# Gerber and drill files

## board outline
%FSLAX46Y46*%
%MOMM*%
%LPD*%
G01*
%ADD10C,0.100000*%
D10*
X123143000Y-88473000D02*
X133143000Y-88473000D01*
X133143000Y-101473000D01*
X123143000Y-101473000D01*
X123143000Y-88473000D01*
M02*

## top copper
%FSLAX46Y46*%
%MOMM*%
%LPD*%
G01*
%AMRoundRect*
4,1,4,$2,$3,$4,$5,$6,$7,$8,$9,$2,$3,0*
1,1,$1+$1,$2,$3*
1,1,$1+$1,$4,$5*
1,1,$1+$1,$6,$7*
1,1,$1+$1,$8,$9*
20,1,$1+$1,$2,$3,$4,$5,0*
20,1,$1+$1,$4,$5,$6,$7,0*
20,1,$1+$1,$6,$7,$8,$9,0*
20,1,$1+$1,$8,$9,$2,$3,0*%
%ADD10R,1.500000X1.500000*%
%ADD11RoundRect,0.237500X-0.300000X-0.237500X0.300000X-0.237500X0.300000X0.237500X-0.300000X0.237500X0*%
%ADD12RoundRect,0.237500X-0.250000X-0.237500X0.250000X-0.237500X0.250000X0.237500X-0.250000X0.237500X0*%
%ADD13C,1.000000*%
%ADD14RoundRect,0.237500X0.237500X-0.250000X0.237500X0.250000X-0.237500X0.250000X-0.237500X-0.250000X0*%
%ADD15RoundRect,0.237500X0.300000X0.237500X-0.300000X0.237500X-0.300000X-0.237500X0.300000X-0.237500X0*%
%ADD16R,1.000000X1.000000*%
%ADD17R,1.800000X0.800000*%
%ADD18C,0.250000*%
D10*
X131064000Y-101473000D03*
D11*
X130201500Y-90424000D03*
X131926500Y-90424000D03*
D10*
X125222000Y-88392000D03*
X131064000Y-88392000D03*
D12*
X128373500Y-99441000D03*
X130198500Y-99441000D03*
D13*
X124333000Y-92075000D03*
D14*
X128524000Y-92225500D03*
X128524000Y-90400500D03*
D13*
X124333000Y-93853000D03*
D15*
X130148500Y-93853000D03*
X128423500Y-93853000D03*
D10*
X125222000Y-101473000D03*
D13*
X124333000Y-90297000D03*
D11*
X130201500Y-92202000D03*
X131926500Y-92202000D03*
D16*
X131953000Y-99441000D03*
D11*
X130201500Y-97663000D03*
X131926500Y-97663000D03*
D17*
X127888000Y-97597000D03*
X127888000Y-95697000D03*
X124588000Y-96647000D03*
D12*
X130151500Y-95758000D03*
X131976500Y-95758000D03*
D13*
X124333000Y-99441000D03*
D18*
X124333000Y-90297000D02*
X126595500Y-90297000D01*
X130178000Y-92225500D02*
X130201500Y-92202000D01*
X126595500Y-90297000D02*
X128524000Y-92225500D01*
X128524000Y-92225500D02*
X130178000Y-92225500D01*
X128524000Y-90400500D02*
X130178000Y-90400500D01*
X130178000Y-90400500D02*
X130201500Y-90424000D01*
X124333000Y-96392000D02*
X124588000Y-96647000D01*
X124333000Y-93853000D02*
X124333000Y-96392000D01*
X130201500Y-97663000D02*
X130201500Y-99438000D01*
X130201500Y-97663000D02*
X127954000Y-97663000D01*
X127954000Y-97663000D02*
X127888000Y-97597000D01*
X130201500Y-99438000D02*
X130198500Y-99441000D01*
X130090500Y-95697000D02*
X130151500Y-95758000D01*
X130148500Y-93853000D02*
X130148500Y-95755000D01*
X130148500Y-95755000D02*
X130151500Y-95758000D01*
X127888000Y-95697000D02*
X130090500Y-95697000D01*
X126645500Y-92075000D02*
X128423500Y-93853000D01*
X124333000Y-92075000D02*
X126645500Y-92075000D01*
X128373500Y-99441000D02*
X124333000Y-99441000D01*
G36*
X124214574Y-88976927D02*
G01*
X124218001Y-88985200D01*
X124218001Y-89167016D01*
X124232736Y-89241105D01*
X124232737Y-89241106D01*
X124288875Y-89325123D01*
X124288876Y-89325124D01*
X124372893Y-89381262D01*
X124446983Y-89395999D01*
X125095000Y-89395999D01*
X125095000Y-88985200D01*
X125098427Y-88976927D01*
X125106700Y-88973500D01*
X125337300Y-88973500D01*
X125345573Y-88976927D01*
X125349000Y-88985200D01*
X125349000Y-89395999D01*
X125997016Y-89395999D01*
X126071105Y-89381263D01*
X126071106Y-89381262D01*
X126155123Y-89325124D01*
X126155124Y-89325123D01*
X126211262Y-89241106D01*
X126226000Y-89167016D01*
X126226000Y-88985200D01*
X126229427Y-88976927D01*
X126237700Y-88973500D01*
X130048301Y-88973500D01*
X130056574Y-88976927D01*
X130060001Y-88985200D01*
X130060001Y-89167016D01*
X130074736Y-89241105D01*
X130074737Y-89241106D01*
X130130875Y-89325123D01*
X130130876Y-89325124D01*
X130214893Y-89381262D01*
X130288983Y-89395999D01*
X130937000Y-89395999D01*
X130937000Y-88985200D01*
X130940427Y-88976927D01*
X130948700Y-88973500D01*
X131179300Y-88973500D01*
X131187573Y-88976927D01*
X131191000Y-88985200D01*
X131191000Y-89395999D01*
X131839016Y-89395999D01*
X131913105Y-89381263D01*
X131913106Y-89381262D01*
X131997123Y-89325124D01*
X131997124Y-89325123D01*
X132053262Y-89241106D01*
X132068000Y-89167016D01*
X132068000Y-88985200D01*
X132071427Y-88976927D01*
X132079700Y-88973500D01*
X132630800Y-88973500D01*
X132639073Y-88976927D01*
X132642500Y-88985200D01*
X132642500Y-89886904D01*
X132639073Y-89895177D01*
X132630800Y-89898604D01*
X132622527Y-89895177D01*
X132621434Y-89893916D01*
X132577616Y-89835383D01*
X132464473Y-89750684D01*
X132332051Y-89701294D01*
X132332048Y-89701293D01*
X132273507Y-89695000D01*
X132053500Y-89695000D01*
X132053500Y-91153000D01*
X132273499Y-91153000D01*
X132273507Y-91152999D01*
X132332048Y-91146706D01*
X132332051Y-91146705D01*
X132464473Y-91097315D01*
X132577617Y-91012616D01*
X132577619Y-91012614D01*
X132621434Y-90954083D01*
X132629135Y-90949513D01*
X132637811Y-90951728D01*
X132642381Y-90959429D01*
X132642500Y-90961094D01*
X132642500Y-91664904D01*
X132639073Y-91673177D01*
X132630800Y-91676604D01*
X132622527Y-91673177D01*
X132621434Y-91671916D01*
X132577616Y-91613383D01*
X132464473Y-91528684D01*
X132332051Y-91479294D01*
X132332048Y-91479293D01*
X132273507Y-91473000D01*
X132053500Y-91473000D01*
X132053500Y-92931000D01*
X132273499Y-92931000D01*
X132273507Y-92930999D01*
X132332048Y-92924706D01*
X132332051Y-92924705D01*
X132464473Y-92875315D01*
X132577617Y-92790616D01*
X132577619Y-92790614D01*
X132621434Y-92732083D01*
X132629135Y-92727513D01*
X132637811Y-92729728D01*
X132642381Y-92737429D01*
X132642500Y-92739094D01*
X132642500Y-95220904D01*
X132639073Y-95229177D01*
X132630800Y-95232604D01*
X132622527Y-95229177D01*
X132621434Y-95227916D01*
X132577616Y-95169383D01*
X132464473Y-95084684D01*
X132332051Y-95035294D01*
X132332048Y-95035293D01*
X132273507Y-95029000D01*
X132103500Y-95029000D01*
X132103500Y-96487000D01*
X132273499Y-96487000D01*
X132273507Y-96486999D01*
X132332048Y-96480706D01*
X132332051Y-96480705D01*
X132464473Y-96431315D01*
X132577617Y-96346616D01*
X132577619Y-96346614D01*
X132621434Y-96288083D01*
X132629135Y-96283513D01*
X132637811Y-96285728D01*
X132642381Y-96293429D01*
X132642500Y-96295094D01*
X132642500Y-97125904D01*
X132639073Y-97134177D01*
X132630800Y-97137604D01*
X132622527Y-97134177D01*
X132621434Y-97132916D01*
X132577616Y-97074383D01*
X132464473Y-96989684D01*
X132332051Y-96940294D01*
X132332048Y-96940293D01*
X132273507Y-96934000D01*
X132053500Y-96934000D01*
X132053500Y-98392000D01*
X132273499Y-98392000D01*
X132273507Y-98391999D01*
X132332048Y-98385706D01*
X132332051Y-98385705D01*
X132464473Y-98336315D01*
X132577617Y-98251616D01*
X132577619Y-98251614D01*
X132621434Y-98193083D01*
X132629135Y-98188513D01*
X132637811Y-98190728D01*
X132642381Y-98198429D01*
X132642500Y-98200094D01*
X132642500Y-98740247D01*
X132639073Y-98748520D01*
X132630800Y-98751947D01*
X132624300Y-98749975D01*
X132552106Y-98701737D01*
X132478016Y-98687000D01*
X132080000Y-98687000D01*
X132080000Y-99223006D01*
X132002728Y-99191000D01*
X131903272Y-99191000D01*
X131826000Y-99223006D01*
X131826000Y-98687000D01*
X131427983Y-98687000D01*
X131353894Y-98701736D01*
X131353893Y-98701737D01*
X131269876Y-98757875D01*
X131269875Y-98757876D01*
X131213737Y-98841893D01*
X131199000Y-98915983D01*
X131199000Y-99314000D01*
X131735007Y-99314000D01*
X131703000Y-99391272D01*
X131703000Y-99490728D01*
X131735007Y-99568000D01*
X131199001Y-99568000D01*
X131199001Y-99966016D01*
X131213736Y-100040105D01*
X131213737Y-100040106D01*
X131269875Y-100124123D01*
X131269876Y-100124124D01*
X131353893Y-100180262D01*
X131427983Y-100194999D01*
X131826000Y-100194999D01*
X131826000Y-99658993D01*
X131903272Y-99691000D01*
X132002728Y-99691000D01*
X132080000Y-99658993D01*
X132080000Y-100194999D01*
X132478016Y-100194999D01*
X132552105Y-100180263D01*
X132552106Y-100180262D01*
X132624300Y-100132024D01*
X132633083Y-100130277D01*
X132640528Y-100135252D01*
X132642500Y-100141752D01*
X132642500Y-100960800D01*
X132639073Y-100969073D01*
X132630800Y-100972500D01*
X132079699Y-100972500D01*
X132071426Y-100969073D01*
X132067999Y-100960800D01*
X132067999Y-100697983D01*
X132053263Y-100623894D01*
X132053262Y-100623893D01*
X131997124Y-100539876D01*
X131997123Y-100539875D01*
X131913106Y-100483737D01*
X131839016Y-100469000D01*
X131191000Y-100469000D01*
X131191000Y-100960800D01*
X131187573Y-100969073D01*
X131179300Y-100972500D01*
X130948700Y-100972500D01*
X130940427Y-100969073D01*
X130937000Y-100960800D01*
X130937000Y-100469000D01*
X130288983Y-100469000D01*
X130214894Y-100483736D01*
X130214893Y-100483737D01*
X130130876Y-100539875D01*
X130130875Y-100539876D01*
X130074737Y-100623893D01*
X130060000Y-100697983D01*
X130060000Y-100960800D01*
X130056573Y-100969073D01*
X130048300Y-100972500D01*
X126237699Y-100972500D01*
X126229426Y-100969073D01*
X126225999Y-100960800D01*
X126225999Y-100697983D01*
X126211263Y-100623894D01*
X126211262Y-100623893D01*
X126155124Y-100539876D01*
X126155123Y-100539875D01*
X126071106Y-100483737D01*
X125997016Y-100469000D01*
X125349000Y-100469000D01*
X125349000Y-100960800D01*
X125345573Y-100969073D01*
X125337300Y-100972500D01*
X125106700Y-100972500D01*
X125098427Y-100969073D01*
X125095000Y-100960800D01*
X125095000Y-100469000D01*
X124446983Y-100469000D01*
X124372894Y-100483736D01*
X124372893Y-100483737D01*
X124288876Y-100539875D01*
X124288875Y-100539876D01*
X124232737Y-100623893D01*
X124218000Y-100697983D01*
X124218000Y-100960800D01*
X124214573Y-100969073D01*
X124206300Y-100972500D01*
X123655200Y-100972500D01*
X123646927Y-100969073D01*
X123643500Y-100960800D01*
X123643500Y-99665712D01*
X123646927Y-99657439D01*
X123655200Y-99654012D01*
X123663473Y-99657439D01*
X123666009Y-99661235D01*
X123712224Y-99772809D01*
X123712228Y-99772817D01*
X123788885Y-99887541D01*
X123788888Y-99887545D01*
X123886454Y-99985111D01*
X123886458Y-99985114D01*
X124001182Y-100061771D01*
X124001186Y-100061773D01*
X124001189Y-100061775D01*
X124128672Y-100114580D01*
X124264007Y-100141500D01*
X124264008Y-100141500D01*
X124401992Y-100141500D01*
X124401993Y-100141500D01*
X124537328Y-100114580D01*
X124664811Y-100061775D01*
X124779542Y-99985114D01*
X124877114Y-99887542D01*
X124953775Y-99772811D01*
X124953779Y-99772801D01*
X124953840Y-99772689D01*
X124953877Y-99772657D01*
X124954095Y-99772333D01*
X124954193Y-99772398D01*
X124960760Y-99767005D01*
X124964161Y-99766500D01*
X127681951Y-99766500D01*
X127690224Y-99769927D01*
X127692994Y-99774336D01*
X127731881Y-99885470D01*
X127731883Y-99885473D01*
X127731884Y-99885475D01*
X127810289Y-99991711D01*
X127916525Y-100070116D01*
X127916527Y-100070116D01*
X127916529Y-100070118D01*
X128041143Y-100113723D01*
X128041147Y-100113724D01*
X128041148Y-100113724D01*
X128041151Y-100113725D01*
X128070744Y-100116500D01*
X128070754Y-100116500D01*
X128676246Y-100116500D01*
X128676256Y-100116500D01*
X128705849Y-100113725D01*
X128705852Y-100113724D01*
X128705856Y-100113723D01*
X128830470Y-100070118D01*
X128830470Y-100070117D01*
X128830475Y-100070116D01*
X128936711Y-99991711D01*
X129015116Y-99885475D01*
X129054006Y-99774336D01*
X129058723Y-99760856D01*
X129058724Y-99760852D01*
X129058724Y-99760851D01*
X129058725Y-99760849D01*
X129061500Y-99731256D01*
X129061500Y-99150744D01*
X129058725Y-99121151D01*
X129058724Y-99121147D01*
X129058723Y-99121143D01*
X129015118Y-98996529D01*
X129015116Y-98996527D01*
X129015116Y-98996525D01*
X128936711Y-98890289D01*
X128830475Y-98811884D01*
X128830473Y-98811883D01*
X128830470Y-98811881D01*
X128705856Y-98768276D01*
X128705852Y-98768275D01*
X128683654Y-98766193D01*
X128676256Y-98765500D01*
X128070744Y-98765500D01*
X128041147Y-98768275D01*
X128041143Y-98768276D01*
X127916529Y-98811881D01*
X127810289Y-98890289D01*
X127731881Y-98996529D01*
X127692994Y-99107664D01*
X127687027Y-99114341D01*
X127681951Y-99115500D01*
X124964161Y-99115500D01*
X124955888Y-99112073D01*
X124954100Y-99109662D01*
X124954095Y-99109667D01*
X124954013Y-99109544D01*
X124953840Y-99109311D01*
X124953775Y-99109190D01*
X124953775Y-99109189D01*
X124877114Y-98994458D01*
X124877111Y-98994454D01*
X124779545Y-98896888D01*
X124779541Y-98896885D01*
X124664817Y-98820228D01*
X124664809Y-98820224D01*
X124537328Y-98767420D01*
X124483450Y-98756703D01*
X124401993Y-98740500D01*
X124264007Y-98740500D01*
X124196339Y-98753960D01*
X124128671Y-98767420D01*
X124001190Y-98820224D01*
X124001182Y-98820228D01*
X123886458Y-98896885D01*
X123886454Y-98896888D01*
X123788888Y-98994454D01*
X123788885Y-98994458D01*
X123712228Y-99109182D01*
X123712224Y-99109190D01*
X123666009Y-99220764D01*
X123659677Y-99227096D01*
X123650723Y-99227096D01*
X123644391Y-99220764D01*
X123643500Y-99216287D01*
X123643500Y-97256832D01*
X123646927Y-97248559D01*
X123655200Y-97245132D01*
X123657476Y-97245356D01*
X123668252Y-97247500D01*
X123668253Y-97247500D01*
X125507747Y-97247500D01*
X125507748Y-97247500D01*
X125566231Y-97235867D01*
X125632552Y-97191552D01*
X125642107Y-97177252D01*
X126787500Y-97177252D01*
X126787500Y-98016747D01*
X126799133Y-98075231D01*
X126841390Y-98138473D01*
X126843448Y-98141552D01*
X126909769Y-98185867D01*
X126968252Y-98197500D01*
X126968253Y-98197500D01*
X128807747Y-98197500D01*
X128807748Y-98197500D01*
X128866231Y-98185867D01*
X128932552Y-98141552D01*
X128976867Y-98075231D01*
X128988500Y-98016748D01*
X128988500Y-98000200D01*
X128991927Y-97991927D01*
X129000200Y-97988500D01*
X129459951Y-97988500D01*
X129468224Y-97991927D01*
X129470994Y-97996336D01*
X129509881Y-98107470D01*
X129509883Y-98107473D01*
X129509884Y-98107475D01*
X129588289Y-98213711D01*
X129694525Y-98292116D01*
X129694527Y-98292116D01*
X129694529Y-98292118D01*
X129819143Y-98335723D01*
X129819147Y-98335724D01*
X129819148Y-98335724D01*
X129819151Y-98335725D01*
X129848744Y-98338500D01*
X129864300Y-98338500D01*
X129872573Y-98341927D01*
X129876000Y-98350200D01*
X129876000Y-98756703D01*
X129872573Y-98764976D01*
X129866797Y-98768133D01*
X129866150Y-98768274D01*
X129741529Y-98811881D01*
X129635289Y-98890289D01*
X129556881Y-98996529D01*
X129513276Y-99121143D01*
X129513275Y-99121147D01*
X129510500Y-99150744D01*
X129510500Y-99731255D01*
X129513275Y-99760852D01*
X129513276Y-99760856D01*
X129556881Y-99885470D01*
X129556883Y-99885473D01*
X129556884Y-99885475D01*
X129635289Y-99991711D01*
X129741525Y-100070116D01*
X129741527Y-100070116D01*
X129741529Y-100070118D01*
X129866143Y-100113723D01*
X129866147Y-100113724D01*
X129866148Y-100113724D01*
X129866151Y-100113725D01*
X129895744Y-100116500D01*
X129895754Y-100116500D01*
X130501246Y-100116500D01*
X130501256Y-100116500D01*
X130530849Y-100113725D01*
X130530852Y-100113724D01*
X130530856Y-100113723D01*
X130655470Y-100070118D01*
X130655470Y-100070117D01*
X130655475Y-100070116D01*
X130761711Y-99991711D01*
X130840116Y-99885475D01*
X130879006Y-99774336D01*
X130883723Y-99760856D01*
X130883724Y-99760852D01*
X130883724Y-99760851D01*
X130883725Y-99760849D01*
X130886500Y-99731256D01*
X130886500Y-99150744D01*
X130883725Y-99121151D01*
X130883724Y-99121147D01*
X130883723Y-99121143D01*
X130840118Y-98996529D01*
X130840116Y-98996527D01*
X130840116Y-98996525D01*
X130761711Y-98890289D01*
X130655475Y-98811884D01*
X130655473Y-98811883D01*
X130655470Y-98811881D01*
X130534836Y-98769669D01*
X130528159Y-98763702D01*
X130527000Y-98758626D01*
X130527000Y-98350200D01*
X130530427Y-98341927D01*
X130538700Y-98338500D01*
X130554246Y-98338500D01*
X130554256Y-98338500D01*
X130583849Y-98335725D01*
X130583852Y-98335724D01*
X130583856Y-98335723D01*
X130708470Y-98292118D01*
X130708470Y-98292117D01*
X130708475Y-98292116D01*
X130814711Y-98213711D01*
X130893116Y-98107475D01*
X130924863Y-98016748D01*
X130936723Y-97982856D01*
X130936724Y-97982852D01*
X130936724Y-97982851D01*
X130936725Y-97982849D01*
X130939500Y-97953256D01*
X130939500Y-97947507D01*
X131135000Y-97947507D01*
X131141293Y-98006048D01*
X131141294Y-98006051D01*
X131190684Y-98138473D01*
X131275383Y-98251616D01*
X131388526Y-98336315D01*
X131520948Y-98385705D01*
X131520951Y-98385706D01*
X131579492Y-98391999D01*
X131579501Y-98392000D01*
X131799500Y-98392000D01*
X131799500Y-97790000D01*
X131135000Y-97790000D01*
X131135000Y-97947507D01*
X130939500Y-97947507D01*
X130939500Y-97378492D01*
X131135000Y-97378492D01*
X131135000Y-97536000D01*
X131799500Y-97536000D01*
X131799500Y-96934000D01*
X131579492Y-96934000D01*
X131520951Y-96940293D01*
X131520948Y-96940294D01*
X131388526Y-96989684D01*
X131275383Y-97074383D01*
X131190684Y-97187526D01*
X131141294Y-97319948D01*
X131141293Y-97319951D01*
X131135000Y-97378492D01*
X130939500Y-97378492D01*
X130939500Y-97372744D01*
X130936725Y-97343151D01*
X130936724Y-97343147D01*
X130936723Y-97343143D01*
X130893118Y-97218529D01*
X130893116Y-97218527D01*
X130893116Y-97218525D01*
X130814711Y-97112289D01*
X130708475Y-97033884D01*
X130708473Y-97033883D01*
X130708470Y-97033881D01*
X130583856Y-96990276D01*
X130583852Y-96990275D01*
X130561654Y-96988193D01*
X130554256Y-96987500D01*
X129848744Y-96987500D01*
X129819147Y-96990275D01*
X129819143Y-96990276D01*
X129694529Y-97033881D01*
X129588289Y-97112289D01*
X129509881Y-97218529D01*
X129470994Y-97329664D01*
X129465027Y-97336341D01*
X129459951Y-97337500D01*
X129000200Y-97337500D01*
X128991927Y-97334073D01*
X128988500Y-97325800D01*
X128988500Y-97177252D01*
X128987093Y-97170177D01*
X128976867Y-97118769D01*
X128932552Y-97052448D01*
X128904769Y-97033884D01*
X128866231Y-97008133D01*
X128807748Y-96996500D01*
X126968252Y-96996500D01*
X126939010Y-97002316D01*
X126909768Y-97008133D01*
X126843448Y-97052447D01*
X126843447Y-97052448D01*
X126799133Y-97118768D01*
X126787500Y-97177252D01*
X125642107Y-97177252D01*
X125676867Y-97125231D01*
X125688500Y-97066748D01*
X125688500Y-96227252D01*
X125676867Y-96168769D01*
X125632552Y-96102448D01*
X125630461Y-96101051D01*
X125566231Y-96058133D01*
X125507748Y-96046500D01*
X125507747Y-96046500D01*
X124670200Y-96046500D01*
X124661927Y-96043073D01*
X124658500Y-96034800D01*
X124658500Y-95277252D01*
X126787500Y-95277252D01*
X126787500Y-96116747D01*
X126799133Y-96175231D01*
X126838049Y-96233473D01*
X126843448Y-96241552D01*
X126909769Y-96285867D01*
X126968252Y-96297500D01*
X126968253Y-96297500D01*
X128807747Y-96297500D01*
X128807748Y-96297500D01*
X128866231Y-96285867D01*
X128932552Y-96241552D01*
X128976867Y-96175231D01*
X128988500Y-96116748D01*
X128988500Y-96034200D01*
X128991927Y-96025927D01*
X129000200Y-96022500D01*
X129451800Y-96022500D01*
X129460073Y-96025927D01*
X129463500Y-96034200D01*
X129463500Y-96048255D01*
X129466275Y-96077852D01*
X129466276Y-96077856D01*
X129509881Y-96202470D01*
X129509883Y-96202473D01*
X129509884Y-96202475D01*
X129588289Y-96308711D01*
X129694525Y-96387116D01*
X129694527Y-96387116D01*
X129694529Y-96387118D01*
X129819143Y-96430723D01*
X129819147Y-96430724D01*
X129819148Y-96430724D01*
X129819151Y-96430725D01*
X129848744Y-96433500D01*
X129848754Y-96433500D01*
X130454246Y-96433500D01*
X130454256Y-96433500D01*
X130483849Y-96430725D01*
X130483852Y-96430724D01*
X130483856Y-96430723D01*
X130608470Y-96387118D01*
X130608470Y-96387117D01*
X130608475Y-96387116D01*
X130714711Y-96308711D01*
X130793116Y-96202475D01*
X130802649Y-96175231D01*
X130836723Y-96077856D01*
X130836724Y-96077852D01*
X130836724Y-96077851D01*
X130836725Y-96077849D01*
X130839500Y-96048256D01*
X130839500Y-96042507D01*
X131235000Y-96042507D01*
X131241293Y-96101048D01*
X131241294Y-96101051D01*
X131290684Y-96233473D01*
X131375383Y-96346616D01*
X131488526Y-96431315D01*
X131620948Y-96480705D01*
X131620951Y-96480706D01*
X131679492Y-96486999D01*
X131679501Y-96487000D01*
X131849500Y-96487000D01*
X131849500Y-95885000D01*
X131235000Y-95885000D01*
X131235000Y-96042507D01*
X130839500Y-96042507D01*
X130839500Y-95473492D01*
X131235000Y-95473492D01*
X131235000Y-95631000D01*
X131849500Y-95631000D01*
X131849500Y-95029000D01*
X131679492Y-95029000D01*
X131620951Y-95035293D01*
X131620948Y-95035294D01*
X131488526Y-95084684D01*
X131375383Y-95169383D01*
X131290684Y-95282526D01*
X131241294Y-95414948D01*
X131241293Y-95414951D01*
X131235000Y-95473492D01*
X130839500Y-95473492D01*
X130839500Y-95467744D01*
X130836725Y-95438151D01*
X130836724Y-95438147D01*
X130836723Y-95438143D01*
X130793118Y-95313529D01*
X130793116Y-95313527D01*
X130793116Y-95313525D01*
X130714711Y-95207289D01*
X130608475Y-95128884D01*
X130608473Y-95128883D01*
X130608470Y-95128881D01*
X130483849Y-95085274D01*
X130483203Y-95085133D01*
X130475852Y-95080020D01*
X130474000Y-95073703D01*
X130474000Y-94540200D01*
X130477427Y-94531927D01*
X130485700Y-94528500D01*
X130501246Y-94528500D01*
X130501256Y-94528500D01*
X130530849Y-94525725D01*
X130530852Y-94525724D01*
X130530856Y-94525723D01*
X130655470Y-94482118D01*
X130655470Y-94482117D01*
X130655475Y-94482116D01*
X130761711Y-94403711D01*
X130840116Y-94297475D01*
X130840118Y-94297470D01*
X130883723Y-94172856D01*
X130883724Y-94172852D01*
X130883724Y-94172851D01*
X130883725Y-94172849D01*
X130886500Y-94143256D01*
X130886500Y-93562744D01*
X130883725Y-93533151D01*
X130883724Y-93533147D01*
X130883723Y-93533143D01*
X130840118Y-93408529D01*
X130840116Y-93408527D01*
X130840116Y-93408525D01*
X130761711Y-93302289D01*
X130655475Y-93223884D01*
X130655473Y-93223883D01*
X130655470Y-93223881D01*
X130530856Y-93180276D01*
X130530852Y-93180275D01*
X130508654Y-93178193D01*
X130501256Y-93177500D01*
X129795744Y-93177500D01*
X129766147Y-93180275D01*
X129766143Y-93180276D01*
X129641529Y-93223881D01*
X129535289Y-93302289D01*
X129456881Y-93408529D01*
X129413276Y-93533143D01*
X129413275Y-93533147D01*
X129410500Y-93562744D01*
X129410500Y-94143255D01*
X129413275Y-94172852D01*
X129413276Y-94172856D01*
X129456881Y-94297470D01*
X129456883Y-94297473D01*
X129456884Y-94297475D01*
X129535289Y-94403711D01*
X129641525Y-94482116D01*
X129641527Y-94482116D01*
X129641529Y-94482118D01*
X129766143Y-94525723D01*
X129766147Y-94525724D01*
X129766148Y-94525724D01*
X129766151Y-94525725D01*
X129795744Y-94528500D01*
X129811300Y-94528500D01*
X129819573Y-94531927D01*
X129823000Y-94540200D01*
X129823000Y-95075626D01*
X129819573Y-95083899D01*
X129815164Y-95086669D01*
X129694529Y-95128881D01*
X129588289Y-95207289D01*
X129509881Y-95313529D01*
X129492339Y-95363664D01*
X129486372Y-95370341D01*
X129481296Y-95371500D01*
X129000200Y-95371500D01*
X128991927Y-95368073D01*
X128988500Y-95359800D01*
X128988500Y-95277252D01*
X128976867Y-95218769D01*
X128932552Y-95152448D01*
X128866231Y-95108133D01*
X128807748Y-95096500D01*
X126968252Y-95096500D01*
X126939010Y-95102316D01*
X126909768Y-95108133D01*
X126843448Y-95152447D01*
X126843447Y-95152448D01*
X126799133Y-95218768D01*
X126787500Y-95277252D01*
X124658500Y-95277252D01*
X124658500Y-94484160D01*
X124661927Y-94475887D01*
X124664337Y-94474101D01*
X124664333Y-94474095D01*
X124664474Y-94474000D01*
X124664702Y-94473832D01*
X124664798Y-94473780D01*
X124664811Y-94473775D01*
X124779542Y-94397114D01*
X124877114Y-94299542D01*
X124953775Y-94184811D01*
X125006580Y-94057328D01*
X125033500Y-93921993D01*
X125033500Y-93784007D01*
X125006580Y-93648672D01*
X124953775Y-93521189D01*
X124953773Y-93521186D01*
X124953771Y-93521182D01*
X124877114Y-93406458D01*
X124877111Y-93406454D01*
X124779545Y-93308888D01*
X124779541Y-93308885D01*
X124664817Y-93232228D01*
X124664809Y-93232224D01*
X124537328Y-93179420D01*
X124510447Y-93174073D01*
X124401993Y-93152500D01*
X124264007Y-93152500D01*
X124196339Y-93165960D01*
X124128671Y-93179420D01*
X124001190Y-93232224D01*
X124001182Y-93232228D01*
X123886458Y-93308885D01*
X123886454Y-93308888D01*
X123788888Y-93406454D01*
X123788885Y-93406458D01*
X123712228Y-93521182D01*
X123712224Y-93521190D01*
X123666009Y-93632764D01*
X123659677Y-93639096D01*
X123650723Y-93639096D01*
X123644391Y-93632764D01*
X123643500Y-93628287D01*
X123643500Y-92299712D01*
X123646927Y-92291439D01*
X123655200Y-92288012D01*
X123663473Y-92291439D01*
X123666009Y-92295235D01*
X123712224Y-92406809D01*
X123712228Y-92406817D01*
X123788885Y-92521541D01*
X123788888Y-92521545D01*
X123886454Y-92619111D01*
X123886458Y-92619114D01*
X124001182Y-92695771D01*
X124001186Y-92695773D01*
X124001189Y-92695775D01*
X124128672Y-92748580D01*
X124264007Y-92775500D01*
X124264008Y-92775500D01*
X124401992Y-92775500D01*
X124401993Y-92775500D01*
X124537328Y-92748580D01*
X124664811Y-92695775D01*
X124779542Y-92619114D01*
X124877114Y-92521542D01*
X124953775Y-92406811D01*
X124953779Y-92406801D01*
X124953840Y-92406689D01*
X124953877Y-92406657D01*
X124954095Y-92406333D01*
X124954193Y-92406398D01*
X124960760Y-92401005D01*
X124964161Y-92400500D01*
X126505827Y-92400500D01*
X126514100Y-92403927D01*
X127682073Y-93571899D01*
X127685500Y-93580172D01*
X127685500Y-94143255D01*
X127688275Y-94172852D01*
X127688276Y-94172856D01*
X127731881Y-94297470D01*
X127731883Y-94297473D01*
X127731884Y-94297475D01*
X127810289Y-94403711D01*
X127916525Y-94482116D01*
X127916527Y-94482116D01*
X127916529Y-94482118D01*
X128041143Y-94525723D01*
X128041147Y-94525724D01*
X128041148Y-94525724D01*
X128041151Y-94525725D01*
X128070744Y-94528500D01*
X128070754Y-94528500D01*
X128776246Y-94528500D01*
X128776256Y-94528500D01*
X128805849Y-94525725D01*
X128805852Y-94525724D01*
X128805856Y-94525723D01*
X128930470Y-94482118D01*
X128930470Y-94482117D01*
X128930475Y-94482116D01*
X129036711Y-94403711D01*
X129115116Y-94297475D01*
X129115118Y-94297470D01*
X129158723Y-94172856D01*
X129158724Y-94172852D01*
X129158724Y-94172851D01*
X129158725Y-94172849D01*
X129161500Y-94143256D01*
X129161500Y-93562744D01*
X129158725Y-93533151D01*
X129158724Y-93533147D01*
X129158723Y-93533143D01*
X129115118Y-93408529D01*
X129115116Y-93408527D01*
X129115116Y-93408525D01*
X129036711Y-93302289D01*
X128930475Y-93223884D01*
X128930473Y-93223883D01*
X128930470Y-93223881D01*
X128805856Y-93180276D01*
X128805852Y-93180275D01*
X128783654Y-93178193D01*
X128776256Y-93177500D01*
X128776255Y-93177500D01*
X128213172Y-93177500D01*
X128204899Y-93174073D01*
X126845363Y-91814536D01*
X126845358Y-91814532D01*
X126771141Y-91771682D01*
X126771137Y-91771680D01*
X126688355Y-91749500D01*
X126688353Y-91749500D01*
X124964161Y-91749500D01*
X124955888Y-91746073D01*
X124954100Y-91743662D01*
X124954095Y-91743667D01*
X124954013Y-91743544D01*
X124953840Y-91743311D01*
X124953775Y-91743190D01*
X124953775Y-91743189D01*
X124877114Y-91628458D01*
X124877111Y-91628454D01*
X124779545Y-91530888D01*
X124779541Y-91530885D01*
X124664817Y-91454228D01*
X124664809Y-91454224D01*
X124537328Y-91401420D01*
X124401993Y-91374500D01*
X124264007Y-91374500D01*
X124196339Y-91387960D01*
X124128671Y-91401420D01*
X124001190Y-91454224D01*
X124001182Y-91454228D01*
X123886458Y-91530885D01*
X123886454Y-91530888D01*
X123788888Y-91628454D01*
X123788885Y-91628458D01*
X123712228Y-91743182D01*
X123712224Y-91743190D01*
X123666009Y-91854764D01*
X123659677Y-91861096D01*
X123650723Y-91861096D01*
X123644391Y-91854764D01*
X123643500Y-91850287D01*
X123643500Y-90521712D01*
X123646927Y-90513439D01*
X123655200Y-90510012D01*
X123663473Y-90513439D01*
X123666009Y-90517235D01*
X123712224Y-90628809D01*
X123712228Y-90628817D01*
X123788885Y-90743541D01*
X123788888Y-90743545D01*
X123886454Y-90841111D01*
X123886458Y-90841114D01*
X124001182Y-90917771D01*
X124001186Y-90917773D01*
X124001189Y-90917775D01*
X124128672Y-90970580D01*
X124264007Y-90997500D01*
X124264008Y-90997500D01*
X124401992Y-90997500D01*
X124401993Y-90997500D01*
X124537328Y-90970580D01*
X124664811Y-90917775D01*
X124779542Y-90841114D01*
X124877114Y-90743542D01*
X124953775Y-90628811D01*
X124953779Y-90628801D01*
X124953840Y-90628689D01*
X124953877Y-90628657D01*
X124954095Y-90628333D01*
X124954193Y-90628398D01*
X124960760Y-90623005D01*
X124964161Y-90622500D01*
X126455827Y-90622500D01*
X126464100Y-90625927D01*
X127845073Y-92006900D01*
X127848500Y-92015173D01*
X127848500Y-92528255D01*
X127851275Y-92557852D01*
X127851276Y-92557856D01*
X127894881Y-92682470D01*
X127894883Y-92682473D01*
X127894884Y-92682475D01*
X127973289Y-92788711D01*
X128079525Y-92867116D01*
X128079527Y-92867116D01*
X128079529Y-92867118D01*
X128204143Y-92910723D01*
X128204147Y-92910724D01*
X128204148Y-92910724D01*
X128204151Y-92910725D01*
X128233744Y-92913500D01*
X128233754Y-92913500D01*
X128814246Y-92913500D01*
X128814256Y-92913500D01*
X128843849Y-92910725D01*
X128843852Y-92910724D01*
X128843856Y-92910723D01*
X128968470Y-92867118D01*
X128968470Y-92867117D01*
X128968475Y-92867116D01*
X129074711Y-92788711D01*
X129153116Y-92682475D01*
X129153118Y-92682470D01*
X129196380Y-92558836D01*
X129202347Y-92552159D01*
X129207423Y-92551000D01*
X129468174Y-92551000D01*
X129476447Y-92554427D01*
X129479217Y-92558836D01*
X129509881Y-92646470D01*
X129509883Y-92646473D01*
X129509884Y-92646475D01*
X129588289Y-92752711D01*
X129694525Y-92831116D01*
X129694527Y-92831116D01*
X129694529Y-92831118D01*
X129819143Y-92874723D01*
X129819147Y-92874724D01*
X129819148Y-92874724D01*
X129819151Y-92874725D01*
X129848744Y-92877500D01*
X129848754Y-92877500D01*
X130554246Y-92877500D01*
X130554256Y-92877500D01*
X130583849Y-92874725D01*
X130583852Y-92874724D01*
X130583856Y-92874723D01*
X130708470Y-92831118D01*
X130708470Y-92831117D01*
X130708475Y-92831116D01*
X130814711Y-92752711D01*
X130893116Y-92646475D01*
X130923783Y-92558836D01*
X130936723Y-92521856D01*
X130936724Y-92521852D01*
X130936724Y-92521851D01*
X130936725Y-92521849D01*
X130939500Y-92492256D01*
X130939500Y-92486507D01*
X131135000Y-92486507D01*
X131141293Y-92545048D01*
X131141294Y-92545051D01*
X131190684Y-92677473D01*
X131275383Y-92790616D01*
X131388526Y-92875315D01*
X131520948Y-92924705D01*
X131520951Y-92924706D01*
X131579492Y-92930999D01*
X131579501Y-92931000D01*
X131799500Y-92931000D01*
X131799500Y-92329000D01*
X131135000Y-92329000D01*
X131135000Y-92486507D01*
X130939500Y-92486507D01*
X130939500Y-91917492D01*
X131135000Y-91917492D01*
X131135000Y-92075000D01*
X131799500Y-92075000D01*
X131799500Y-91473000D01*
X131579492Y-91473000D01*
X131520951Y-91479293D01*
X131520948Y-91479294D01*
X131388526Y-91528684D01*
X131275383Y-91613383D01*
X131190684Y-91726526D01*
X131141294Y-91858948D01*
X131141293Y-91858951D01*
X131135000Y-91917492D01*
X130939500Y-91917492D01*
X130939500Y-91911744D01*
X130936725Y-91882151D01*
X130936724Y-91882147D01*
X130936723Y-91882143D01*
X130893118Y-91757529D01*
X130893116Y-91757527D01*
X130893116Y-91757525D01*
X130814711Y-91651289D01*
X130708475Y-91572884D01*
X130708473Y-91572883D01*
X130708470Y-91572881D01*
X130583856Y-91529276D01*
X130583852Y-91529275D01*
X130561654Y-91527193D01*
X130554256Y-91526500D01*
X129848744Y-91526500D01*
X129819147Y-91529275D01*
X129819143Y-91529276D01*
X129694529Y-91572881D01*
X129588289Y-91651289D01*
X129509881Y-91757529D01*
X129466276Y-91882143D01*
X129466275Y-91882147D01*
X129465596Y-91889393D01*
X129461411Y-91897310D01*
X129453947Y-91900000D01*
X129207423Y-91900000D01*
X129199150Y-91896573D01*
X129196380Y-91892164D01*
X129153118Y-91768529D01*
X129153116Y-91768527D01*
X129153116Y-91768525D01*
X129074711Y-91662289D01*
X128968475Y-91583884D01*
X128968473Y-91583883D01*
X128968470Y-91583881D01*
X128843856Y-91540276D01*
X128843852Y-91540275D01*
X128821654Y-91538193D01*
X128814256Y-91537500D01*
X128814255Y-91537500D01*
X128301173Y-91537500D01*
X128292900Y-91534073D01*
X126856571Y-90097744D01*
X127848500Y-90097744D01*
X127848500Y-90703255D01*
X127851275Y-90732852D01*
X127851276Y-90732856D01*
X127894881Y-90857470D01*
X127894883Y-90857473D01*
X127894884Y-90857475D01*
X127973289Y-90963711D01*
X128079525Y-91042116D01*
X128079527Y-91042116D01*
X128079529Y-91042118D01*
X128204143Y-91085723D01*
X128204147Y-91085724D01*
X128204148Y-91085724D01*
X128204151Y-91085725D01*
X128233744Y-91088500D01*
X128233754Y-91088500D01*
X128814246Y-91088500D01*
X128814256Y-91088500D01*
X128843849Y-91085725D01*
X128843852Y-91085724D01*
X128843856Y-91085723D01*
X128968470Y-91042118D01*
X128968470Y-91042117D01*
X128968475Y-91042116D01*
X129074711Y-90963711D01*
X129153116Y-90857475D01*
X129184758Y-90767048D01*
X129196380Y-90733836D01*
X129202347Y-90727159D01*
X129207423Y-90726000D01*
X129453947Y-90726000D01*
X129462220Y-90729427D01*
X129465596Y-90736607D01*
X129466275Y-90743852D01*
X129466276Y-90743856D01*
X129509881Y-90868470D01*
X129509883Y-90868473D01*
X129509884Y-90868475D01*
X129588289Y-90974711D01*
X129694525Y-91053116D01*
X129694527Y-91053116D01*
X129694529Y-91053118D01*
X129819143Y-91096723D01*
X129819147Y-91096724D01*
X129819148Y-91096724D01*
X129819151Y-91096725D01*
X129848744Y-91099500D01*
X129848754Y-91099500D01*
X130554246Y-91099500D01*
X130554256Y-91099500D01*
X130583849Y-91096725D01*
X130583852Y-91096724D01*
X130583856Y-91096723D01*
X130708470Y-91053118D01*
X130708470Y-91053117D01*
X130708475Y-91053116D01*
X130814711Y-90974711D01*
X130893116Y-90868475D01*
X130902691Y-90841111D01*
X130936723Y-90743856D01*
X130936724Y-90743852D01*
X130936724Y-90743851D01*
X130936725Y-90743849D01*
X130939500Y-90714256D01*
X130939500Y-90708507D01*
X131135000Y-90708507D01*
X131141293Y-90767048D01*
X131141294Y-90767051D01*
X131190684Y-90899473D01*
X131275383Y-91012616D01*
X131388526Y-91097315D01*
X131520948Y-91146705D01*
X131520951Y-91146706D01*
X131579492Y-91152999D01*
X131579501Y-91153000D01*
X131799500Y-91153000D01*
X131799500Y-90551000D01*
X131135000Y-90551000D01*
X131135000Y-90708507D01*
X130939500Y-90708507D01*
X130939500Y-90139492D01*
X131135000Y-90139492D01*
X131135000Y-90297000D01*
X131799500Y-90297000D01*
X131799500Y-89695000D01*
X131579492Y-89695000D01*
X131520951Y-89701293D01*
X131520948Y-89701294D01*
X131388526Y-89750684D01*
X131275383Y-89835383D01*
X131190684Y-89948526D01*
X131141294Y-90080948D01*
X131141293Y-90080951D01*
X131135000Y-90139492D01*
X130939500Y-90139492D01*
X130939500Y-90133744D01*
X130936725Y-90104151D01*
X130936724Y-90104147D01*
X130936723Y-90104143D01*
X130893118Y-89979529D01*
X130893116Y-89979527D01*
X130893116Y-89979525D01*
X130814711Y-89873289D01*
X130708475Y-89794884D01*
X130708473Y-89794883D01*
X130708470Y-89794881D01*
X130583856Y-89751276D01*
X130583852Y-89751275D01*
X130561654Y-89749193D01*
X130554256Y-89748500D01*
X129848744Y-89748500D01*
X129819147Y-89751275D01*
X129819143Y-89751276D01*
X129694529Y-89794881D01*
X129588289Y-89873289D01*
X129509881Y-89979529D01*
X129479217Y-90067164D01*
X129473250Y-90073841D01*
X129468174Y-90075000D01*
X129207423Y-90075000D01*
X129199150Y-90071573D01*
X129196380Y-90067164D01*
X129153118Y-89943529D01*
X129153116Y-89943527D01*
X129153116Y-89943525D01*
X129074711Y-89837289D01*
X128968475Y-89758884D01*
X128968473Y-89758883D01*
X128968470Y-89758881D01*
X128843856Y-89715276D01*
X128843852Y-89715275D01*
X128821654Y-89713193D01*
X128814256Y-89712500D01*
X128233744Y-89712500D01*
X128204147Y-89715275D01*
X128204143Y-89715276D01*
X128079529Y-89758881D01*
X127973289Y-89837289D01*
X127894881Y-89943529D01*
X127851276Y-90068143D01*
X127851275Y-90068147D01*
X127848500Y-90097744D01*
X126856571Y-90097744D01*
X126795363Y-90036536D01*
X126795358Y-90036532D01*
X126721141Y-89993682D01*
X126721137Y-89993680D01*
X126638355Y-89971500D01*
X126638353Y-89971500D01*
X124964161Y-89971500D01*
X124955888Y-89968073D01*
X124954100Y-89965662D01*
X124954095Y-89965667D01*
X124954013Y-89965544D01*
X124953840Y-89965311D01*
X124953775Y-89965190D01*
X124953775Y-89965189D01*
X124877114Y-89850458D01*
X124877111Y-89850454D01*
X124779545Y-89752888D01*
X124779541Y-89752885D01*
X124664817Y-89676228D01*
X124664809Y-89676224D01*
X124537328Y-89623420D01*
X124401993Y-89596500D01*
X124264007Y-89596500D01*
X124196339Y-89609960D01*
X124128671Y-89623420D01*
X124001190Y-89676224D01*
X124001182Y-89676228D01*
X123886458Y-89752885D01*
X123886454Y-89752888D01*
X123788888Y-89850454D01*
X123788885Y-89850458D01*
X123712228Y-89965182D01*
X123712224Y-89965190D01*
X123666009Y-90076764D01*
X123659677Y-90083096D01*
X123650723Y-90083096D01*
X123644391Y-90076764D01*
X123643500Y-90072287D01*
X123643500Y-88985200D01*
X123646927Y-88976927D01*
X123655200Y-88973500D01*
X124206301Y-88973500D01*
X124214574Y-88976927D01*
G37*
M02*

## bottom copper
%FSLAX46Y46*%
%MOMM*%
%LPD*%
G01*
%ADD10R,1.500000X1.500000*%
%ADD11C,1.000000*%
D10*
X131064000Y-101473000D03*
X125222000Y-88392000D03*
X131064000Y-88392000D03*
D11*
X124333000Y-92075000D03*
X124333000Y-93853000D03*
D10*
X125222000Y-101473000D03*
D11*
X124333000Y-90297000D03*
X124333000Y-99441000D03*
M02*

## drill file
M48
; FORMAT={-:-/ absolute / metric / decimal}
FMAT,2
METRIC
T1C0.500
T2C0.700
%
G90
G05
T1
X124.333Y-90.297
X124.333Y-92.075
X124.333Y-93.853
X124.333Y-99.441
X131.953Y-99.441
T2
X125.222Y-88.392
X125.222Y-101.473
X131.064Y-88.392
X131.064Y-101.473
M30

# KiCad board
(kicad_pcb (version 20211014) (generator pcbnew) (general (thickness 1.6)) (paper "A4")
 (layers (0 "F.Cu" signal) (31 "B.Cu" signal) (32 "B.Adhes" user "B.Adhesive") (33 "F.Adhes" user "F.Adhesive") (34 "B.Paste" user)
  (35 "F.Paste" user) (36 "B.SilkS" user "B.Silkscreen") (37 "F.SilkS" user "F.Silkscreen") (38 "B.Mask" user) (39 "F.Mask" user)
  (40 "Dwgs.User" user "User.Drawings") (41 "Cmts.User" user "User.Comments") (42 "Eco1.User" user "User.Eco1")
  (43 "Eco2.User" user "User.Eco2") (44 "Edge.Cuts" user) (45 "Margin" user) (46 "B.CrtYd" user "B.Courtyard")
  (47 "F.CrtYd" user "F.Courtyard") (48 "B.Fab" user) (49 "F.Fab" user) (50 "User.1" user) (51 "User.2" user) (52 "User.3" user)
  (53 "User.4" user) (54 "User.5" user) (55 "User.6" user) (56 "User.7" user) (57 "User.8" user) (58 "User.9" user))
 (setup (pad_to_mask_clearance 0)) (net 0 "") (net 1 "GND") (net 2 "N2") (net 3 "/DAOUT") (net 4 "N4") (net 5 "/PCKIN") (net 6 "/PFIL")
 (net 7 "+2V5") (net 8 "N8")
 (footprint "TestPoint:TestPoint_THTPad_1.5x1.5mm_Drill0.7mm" (layer "F.Cu") (at 131.064 101.473)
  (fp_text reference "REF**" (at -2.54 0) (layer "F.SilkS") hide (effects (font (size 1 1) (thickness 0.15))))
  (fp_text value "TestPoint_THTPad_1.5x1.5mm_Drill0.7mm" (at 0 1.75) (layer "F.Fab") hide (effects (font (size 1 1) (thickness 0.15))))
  (pad "1" thru_hole rect (at 0 0) (size 1.5 1.5) (drill 0.7) (layers *.Cu *.Mask) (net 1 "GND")))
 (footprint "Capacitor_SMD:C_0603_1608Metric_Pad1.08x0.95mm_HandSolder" (layer "F.Cu") (at 131.064 90.424)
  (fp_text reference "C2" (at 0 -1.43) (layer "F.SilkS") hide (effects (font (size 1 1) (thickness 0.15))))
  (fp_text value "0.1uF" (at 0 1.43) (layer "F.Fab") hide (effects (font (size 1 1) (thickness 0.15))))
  (pad "1" smd roundrect (at -0.8625 0) (size 1.075 0.95) (layers "F.Cu" "F.Paste" "F.Mask") (roundrect_rratio 0.25) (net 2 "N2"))
  (pad "2" smd roundrect (at 0.8625 0) (size 1.075 0.95) (layers "F.Cu" "F.Paste" "F.Mask") (roundrect_rratio 0.25) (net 1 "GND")))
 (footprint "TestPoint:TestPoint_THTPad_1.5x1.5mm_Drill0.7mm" (layer "F.Cu") (at 125.222 88.392)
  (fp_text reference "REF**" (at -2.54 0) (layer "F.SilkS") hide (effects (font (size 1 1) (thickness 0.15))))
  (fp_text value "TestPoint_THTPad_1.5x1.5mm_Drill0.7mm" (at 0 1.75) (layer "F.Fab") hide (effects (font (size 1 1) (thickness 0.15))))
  (pad "1" thru_hole rect (at 0 0) (size 1.5 1.5) (drill 0.7) (layers *.Cu *.Mask) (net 1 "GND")))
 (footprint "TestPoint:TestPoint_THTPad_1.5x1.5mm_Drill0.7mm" (layer "F.Cu") (at 131.064 88.392)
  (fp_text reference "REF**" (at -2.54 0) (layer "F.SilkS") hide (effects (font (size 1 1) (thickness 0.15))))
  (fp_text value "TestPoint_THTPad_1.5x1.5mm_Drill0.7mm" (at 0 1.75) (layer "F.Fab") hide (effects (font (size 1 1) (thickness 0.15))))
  (pad "1" thru_hole rect (at 0 0) (size 1.5 1.5) (drill 0.7) (layers *.Cu *.Mask) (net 1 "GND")))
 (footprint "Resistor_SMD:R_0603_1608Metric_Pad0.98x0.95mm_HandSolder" (layer "F.Cu") (at 129.286 99.441)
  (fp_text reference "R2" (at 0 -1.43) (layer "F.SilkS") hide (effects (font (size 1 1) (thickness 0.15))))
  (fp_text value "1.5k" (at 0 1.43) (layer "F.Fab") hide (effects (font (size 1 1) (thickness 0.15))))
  (pad "1" smd roundrect (at -0.9125 0) (size 0.975 0.95) (layers "F.Cu" "F.Paste" "F.Mask") (roundrect_rratio 0.25) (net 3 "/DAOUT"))
  (pad "2" smd roundrect (at 0.9125 0) (size 0.975 0.95) (layers "F.Cu" "F.Paste" "F.Mask") (roundrect_rratio 0.25) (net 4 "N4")))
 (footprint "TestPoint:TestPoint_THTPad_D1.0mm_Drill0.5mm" (layer "F.Cu") (at 124.333 92.075)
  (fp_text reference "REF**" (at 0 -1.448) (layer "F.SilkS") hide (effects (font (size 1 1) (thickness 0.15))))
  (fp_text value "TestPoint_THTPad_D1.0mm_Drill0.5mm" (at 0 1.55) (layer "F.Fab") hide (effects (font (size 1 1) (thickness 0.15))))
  (pad "1" thru_hole circle (at 0 0) (size 1 1) (drill 0.5) (layers *.Cu *.Mask) (remove_unused_layers) (keep_end_layers) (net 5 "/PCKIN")))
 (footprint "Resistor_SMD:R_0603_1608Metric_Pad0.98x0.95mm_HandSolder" (layer "F.Cu") (at 128.524 91.313 90)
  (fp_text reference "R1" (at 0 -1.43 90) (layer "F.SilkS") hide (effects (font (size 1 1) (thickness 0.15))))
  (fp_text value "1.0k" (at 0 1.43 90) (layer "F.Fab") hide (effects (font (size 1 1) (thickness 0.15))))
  (pad "1" smd roundrect (at -0.9125 0 90) (size 0.975 0.95) (layers "F.Cu" "F.Paste" "F.Mask") (roundrect_rratio 0.25) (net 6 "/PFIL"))
  (pad "2" smd roundrect (at 0.9125 0 90) (size 0.975 0.95) (layers "F.Cu" "F.Paste" "F.Mask") (roundrect_rratio 0.25) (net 2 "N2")))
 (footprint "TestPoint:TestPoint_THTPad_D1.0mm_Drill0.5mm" (layer "F.Cu") (at 124.333 93.853)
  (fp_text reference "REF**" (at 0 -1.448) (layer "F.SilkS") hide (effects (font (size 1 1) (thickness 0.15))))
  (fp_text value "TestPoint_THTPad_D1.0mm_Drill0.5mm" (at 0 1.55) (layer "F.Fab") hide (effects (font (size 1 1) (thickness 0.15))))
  (pad "1" thru_hole circle (at 0 0) (size 1 1) (drill 0.5) (layers *.Cu *.Mask) (remove_unused_layers) (keep_end_layers) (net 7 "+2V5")))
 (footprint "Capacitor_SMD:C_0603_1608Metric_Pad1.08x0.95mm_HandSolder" (layer "F.Cu") (at 129.286 93.853 180)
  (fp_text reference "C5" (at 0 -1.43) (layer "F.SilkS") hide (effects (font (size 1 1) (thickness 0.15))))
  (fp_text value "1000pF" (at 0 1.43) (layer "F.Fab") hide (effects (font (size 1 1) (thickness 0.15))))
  (pad "1" smd roundrect (at -0.8625 0 180) (size 1.075 0.95) (layers "F.Cu" "F.Paste" "F.Mask") (roundrect_rratio 0.25) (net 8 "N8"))
  (pad "2" smd roundrect (at 0.8625 0 180) (size 1.075 0.95) (layers "F.Cu" "F.Paste" "F.Mask") (roundrect_rratio 0.25) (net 5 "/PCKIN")))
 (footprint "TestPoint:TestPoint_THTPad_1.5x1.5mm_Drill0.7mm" (layer "F.Cu") (at 125.222 101.473)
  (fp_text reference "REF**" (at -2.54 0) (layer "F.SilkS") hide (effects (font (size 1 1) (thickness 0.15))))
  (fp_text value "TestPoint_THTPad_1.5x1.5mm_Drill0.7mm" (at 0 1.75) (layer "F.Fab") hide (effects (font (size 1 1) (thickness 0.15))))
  (pad "1" thru_hole rect (at 0 0) (size 1.5 1.5) (drill 0.7) (layers *.Cu *.Mask) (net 1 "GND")))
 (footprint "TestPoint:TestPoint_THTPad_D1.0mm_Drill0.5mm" (layer "F.Cu") (at 124.333 90.297)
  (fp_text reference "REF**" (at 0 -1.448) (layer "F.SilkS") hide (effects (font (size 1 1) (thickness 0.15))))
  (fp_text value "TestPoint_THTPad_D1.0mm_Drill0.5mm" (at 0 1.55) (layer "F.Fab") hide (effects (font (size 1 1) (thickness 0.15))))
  (pad "1" thru_hole circle (at 0 0) (size 1 1) (drill 0.5) (layers *.Cu *.Mask) (remove_unused_layers) (keep_end_layers) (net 6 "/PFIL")))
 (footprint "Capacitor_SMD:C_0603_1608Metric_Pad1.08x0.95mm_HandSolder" (layer "F.Cu") (at 131.064 92.202)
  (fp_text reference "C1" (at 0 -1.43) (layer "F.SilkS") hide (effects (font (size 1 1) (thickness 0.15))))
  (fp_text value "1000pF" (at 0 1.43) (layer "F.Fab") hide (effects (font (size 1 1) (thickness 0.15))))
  (pad "1" smd roundrect (at -0.8625 0) (size 1.075 0.95) (layers "F.Cu" "F.Paste" "F.Mask") (roundrect_rratio 0.25) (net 6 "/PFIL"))
  (pad "2" smd roundrect (at 0.8625 0) (size 1.075 0.95) (layers "F.Cu" "F.Paste" "F.Mask") (roundrect_rratio 0.25) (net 1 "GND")))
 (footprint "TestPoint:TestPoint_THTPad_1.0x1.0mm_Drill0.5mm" (layer "F.Cu") (at 131.953 99.441)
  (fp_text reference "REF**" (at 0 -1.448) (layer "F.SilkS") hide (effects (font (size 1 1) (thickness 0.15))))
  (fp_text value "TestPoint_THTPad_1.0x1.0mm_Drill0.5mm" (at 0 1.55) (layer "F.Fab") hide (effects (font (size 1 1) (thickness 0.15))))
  (pad "1" thru_hole rect (at 0 0) (size 1 1) (drill 0.5) (layers *.Cu *.Mask) (remove_unused_layers) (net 1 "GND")))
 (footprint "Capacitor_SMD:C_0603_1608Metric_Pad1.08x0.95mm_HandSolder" (layer "F.Cu") (at 131.064 97.663)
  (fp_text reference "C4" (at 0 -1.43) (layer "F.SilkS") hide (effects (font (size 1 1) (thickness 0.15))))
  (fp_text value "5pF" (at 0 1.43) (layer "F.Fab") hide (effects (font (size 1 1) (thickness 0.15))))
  (pad "1" smd roundrect (at -0.8625 0) (size 1.075 0.95) (layers "F.Cu" "F.Paste" "F.Mask") (roundrect_rratio 0.25) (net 4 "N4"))
  (pad "2" smd roundrect (at 0.8625 0) (size 1.075 0.95) (layers "F.Cu" "F.Paste" "F.Mask") (roundrect_rratio 0.25) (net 1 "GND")))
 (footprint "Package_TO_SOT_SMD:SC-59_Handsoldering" (layer "F.Cu") (at 126.238 96.647 180)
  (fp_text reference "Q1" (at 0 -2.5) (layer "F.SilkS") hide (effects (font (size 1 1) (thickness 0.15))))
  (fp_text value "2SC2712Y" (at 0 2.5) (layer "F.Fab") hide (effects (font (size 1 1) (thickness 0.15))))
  (pad "1" smd rect (at -1.65 -0.95 180) (size 1.8 0.8) (layers "F.Cu" "F.Paste" "F.Mask") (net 4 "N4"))
  (pad "2" smd rect (at -1.65 0.95 180) (size 1.8 0.8) (layers "F.Cu" "F.Paste" "F.Mask") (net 8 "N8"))
  (pad "3" smd rect (at 1.65 0 180) (size 1.8 0.8) (layers "F.Cu" "F.Paste" "F.Mask") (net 7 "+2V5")))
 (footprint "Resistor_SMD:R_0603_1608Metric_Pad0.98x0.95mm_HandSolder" (layer "F.Cu") (at 131.064 95.758)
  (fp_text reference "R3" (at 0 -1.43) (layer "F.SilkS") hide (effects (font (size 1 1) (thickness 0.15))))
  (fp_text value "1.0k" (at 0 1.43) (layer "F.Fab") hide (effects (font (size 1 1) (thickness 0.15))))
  (pad "1" smd roundrect (at -0.9125 0) (size 0.975 0.95) (layers "F.Cu" "F.Paste" "F.Mask") (roundrect_rratio 0.25) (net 8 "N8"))
  (pad "2" smd roundrect (at 0.9125 0) (size 0.975 0.95) (layers "F.Cu" "F.Paste" "F.Mask") (roundrect_rratio 0.25) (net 1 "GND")))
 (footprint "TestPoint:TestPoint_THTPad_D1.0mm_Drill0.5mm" (layer "F.Cu") (at 124.333 99.441)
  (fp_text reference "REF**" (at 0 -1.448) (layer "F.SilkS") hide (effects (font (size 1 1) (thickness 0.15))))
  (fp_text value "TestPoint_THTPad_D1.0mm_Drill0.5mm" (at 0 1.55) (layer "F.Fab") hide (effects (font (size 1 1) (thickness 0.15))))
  (pad "1" thru_hole circle (at 0 0) (size 1 1) (drill 0.5) (layers *.Cu *.Mask) (remove_unused_layers) (keep_end_layers) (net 3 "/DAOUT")))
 (gr_rect (start 133.143 101.473) (end 123.143 88.473) (layer "Edge.Cuts") (width 0.1) (fill none))
 (segment (start 124.333 90.297) (end 126.5955 90.297) (width 0.25) (layer "F.Cu") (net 6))
 (segment (start 130.178 92.2255) (end 130.2015 92.202) (width 0.25) (layer "F.Cu") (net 6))
 (segment (start 126.5955 90.297) (end 128.524 92.2255) (width 0.25) (layer "F.Cu") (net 6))
 (segment (start 128.524 92.2255) (end 130.178 92.2255) (width 0.25) (layer "F.Cu") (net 6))
 (segment (start 128.524 90.4005) (end 130.178 90.4005) (width 0.25) (layer "F.Cu") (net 2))
 (segment (start 130.178 90.4005) (end 130.2015 90.424) (width 0.25) (layer "F.Cu") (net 2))
 (segment (start 124.333 96.392) (end 124.588 96.647) (width 0.25) (layer "F.Cu") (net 7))
 (segment (start 124.333 93.853) (end 124.333 96.392) (width 0.25) (layer "F.Cu") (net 7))
 (segment (start 130.2015 97.663) (end 130.2015 99.438) (width 0.25) (layer "F.Cu") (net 4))
 (segment (start 130.2015 97.663) (end 127.954 97.663) (width 0.25) (layer "F.Cu") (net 4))
 (segment (start 127.954 97.663) (end 127.888 97.597) (width 0.25) (layer "F.Cu") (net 4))
 (segment (start 130.2015 99.438) (end 130.1985 99.441) (width 0.25) (layer "F.Cu") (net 4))
 (segment (start 130.0905 95.697) (end 130.1515 95.758) (width 0.25) (layer "F.Cu") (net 8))
 (segment (start 130.1485 93.853) (end 130.1485 95.755) (width 0.25) (layer "F.Cu") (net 8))
 (segment (start 130.1485 95.755) (end 130.1515 95.758) (width 0.25) (layer "F.Cu") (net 8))
 (segment (start 127.888 95.697) (end 130.0905 95.697) (width 0.25) (layer "F.Cu") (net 8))
 (segment (start 126.6455 92.075) (end 128.4235 93.853) (width 0.25) (layer "F.Cu") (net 5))
 (segment (start 124.333 92.075) (end 126.6455 92.075) (width 0.25) (layer "F.Cu") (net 5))
 (segment (start 128.3735 99.441) (end 124.333 99.441) (width 0.25) (layer "F.Cu") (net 3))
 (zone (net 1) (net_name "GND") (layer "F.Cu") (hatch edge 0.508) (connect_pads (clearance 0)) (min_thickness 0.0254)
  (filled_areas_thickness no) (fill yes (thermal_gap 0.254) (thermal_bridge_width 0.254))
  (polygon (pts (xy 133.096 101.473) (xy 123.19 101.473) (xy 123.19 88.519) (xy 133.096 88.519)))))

